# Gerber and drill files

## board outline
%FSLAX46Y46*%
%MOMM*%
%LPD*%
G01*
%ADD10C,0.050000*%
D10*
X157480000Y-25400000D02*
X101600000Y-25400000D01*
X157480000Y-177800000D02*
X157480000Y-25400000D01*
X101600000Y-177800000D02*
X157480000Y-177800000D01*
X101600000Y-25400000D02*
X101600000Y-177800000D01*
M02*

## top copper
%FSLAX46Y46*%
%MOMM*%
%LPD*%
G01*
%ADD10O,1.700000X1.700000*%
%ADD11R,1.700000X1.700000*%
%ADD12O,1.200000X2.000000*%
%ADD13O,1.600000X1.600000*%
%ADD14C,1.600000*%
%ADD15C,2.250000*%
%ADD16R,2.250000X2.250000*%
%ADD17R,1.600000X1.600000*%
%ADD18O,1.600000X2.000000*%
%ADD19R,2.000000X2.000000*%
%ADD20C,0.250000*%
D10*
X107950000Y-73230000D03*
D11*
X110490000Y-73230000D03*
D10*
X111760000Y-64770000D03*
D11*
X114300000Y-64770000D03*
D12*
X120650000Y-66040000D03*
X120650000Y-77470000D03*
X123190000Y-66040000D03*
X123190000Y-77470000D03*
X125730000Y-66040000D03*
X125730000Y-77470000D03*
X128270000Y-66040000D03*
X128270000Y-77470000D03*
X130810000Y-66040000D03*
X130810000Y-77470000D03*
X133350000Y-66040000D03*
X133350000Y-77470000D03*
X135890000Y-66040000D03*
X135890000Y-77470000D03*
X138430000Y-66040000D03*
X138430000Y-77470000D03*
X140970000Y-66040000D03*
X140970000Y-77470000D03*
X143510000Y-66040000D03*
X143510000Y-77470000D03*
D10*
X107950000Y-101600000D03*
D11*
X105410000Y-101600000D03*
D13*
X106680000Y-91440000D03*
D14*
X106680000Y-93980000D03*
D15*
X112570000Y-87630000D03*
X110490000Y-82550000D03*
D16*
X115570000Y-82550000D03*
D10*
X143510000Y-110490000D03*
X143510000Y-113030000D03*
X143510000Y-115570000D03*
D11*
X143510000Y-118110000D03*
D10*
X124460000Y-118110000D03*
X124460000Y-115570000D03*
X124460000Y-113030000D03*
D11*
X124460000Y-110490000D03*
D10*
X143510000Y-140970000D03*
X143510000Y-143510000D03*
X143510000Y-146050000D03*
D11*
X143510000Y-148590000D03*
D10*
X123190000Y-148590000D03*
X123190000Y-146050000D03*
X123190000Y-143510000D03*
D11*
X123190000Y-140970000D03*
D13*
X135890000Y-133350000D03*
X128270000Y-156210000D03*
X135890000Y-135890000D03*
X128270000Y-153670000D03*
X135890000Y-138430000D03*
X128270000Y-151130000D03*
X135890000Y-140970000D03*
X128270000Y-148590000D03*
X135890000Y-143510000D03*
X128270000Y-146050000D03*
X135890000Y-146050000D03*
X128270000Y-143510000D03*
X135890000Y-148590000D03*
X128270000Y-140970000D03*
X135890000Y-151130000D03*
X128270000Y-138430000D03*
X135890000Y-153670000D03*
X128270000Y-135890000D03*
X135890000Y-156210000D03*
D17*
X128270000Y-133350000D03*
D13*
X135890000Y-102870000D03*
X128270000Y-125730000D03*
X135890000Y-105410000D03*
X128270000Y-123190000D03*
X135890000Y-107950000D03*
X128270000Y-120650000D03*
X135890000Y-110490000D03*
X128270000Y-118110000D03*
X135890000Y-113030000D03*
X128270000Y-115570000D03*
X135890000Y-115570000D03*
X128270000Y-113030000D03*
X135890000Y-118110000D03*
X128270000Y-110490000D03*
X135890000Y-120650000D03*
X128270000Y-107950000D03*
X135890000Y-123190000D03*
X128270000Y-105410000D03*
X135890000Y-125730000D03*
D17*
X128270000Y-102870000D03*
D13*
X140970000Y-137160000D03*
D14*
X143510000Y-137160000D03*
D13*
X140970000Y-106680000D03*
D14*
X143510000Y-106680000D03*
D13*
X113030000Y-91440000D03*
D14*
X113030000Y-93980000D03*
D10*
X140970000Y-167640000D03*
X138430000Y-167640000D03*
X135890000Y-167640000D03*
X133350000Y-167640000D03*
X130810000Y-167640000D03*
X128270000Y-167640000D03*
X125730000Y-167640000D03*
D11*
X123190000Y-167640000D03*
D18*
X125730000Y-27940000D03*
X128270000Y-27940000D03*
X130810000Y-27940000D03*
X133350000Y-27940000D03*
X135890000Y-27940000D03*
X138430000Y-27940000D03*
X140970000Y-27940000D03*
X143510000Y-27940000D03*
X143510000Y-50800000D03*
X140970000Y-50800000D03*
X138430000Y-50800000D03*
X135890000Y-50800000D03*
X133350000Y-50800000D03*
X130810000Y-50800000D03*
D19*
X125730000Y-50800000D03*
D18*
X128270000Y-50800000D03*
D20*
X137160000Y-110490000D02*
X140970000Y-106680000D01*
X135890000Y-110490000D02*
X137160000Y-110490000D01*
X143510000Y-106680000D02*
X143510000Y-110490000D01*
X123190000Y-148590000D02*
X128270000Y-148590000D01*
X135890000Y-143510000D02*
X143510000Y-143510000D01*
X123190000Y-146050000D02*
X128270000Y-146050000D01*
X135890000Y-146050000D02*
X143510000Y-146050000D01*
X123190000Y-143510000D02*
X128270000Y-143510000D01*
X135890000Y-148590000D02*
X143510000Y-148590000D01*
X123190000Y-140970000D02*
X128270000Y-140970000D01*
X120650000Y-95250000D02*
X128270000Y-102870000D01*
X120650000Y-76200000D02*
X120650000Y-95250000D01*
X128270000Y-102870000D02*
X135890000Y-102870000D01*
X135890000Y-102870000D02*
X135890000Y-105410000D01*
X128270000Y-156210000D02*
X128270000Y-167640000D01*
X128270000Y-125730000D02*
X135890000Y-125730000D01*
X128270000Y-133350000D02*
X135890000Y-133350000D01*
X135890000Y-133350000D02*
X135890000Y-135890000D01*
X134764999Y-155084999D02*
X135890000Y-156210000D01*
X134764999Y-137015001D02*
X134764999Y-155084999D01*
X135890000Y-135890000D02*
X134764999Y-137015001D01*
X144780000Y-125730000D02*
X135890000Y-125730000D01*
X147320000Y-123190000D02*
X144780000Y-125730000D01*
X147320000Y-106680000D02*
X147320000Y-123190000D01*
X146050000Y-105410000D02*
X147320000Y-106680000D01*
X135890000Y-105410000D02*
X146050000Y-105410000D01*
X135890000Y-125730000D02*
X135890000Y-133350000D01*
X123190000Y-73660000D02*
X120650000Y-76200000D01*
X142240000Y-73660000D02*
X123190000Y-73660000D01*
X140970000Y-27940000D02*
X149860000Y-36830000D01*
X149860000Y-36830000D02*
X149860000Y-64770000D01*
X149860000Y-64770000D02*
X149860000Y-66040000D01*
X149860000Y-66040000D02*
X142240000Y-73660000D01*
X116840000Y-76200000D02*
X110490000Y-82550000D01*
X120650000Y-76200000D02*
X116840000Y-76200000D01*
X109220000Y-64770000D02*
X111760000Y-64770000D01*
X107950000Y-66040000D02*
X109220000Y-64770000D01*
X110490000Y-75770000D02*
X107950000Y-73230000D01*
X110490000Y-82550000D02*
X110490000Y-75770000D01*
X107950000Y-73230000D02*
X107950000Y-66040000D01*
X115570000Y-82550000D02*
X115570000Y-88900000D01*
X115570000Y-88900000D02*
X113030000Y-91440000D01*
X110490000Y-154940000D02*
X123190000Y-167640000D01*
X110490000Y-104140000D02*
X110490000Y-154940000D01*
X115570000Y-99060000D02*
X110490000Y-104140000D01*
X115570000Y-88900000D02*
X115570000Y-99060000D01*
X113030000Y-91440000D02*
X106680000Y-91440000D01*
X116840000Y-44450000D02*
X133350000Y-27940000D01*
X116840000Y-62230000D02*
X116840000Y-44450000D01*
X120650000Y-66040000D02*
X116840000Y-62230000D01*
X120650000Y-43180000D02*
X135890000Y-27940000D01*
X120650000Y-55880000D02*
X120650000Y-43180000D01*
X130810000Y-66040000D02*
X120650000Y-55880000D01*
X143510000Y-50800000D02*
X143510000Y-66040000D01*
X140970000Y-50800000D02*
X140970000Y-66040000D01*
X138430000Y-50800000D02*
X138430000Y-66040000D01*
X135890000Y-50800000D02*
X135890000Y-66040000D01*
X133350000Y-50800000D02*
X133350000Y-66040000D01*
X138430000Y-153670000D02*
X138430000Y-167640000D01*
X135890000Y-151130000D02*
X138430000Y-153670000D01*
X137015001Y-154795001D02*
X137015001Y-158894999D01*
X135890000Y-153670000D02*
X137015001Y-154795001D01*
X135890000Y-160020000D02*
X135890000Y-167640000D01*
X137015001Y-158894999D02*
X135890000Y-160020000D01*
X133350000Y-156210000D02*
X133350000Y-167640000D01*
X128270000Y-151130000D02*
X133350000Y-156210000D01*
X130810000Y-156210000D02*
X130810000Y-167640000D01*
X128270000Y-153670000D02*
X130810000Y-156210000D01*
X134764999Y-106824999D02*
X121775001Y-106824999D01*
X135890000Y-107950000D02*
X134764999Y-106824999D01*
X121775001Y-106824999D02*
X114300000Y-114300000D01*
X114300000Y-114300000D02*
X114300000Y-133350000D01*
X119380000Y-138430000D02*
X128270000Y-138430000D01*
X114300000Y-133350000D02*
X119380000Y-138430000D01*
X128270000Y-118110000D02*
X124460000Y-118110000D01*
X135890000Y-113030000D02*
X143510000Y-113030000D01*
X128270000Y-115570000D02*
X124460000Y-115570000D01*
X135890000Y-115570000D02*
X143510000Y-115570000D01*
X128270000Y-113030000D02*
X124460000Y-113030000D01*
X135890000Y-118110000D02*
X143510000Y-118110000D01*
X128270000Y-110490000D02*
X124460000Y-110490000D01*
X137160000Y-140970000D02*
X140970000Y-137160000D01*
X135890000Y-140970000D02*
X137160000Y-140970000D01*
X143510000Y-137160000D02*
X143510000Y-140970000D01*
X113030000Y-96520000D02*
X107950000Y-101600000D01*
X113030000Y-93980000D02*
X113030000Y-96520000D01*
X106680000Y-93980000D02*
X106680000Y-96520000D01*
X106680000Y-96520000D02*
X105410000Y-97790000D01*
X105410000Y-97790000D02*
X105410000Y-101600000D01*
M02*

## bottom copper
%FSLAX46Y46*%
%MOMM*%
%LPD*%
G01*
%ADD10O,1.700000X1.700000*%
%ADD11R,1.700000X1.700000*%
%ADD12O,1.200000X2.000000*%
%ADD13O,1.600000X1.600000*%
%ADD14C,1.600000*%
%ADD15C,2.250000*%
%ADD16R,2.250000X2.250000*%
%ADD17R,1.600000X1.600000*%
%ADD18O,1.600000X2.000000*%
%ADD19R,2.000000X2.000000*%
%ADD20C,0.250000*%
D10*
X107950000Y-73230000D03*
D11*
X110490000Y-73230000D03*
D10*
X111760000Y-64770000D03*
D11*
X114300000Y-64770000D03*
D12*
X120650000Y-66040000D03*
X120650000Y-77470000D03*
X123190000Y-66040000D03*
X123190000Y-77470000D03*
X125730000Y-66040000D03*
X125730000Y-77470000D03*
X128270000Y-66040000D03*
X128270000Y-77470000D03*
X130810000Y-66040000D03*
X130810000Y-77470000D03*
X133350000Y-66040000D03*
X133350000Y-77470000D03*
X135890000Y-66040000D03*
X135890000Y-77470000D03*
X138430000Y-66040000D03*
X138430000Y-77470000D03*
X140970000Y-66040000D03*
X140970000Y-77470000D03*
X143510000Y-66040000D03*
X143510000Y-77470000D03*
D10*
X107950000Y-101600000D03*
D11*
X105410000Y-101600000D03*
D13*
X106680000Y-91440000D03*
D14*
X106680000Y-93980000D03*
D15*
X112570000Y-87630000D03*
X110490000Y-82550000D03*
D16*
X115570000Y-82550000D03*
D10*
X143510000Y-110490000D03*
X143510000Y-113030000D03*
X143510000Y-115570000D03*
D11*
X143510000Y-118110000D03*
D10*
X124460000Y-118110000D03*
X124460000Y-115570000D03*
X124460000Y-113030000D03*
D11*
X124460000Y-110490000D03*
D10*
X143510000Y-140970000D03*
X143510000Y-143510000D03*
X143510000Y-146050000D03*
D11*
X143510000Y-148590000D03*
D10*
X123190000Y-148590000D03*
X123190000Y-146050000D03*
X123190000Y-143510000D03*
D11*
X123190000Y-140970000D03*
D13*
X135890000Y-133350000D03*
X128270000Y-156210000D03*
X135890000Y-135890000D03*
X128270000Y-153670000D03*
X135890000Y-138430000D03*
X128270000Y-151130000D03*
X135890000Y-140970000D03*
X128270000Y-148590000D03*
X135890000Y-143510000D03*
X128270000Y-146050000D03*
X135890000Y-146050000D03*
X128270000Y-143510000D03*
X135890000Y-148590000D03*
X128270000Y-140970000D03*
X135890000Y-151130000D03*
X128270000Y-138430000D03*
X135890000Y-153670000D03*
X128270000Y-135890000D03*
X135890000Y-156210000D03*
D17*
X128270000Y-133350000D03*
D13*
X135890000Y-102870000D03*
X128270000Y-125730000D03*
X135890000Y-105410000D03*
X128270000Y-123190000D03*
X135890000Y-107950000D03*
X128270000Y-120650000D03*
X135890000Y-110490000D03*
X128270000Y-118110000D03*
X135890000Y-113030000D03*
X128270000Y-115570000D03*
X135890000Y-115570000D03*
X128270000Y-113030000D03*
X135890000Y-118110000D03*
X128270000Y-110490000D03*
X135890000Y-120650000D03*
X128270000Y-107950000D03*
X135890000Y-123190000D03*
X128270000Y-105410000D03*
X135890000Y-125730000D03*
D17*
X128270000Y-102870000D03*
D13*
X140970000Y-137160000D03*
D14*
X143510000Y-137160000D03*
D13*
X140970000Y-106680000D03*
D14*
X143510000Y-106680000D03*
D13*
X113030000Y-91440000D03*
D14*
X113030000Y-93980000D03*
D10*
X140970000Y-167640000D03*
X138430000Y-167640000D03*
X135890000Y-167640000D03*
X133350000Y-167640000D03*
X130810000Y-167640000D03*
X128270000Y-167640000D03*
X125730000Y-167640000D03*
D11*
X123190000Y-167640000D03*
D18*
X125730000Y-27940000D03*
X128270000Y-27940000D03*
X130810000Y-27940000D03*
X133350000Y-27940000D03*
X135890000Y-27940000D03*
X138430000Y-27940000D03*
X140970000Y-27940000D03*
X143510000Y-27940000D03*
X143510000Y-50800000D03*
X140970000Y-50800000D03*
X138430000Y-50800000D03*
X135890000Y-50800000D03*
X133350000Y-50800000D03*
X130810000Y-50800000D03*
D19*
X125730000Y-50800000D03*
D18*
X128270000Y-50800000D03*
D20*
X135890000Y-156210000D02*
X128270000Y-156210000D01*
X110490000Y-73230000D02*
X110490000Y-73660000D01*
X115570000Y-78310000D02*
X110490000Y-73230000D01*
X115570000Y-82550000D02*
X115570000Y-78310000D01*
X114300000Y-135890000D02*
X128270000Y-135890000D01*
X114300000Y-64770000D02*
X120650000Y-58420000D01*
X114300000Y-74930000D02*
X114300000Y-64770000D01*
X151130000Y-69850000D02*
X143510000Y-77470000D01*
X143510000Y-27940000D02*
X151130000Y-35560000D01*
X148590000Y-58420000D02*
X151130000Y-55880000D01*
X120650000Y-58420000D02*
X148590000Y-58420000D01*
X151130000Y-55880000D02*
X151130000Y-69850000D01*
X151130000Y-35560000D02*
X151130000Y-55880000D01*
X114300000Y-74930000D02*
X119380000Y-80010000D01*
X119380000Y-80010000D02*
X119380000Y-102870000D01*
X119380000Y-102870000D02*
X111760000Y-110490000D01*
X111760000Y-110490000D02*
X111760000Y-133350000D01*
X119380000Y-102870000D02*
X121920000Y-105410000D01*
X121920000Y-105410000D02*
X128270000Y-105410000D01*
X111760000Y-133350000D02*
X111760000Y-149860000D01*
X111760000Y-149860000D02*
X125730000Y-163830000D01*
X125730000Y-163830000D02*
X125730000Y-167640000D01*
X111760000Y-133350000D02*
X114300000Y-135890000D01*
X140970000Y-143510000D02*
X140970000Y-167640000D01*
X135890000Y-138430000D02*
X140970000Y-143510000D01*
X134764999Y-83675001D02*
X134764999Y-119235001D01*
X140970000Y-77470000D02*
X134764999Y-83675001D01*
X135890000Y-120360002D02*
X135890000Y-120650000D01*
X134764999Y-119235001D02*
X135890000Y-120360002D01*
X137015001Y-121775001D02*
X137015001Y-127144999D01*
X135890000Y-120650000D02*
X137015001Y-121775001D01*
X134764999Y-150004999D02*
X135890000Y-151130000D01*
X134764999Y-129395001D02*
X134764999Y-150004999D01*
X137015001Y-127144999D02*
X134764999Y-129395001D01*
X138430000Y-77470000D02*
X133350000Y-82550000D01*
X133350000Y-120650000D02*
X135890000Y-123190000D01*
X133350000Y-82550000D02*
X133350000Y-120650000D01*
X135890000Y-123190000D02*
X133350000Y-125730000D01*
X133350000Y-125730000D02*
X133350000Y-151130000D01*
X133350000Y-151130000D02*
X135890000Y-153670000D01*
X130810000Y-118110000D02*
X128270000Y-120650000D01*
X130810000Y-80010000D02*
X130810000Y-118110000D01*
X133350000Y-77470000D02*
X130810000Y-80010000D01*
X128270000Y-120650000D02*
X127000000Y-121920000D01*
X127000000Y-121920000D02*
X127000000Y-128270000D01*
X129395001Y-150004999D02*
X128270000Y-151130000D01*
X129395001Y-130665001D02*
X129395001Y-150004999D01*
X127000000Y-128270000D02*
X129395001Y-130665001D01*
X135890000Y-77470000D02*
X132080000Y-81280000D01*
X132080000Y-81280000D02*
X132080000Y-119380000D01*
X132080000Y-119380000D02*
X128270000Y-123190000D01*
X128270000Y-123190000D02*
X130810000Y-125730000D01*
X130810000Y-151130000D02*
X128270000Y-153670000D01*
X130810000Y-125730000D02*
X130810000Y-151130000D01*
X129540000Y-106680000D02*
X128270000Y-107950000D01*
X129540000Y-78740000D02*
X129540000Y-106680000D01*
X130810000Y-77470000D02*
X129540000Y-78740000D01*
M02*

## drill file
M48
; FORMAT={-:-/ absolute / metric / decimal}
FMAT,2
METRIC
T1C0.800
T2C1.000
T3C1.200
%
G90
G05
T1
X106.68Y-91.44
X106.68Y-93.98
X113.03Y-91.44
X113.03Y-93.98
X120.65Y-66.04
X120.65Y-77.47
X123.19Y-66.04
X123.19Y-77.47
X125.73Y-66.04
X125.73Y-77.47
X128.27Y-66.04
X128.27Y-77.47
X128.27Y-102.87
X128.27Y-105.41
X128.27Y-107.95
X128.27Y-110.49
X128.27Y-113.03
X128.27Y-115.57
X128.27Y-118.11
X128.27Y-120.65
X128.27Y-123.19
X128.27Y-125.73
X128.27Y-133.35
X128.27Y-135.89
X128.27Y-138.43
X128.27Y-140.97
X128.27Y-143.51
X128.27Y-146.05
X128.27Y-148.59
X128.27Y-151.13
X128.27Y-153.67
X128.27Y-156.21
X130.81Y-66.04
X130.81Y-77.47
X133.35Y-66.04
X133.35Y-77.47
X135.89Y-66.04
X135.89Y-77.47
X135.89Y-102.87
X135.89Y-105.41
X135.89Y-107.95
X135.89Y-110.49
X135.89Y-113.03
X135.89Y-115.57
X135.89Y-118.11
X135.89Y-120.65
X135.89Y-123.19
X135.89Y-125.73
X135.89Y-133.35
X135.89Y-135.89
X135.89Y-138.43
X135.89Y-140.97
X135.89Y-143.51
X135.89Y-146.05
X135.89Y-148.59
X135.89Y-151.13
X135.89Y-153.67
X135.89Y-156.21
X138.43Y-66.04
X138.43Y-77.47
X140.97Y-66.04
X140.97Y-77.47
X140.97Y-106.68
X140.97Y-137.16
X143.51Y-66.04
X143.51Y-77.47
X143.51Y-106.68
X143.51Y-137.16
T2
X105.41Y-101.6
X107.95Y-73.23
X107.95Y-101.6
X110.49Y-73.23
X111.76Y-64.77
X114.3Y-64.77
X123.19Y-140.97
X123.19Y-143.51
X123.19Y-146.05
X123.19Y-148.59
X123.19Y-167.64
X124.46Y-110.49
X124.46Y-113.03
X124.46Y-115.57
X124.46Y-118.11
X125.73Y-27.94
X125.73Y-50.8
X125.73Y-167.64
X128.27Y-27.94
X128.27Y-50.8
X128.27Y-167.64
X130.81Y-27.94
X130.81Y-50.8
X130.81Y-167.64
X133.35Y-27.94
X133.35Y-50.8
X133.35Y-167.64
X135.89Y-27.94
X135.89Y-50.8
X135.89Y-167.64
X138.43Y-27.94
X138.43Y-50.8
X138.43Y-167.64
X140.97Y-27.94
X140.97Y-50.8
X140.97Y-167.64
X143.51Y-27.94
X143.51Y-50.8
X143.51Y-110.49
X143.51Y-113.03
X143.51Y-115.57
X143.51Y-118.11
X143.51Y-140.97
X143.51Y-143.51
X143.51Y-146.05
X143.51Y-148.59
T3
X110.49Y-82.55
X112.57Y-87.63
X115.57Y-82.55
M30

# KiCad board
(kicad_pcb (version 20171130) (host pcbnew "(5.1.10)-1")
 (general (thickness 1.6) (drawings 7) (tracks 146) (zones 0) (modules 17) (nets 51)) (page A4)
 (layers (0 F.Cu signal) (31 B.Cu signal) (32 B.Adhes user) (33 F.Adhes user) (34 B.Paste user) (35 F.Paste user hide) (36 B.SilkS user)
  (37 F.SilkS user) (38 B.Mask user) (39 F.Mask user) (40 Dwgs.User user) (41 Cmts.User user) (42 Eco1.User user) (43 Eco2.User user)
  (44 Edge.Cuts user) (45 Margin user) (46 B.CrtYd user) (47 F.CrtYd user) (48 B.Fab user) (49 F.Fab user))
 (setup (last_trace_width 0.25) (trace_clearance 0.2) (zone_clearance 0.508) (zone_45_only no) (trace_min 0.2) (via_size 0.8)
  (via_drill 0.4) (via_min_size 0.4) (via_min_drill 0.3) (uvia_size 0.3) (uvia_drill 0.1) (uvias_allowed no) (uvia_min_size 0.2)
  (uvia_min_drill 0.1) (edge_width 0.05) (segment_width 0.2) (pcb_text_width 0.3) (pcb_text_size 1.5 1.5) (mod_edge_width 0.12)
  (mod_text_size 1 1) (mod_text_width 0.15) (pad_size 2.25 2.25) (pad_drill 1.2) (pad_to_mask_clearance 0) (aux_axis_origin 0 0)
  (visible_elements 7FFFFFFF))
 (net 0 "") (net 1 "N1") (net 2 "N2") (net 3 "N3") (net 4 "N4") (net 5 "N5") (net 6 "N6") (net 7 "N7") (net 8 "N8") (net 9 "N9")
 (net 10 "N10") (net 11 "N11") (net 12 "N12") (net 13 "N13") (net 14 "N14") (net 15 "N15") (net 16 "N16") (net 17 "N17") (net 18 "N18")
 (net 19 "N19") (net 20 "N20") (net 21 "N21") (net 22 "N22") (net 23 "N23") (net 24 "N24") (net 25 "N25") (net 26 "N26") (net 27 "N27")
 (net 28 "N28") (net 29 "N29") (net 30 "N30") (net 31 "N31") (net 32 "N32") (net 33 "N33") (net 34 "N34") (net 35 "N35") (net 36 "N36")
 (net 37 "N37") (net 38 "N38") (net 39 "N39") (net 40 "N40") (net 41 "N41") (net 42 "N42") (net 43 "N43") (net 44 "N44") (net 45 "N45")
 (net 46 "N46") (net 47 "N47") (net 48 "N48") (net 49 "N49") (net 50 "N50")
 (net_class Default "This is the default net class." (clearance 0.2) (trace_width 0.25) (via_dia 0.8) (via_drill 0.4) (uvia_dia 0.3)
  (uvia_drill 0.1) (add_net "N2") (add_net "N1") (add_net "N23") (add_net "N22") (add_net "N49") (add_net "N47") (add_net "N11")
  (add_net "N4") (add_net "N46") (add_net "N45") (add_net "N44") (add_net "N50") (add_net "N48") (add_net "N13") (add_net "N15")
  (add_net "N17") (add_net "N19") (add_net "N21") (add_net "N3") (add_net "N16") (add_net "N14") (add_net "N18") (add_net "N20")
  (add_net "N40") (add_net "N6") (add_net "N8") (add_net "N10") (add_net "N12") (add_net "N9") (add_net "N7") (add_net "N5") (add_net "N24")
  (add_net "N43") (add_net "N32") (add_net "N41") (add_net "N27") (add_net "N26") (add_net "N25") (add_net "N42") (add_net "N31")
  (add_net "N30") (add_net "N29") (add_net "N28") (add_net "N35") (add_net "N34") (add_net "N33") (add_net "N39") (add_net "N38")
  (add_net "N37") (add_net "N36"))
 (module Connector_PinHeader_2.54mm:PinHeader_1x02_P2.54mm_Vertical (layer F.Cu) (at 110.49 73.23 270)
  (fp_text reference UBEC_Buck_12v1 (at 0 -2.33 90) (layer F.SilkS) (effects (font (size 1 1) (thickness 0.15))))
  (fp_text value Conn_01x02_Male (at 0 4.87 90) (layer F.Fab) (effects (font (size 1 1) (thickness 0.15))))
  (pad 2 thru_hole oval (at 0 2.54 270) (size 1.7 1.7) (drill 1) (layers *.Cu *.Mask) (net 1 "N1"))
  (pad 1 thru_hole rect (at 0 0 270) (size 1.7 1.7) (drill 1) (layers *.Cu *.Mask) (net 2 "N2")))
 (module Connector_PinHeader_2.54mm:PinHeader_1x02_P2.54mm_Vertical (layer F.Cu) (at 114.3 64.77 270)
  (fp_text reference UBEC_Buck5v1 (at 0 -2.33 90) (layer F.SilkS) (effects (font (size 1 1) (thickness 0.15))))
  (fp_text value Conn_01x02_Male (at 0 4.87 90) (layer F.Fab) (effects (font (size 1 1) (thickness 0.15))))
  (pad 2 thru_hole oval (at 0 2.54 270) (size 1.7 1.7) (drill 1) (layers *.Cu *.Mask) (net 1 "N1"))
  (pad 1 thru_hole rect (at 0 0 270) (size 1.7 1.7) (drill 1) (layers *.Cu *.Mask) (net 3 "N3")))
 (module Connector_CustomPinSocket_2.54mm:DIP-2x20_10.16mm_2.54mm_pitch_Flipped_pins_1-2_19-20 (layer F.Cu) (at 132.08 64.77 270)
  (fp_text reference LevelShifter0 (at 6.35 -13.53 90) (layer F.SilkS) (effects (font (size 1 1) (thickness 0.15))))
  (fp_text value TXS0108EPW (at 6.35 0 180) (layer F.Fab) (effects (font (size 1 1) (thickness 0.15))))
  (pad 10 thru_hole oval (at 1.27 11.43 180) (size 1.2 2) (drill 0.8) (layers *.Cu *.Mask) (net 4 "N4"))
  (pad 11 thru_hole oval (at 12.7 11.43 180) (size 1.2 2) (drill 0.8) (layers *.Cu *.Mask) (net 1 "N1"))
  (pad 9 thru_hole oval (at 1.27 8.89 180) (size 1.2 2) (drill 0.8) (layers *.Cu *.Mask) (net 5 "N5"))
  (pad 12 thru_hole oval (at 12.7 8.89 180) (size 1.2 2) (drill 0.8) (layers *.Cu *.Mask) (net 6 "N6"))
  (pad 8 thru_hole oval (at 1.27 6.35 180) (size 1.2 2) (drill 0.8) (layers *.Cu *.Mask) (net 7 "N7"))
  (pad 13 thru_hole oval (at 12.7 6.35 180) (size 1.2 2) (drill 0.8) (layers *.Cu *.Mask) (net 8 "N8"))
  (pad 7 thru_hole oval (at 1.27 3.81 180) (size 1.2 2) (drill 0.8) (layers *.Cu *.Mask) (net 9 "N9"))
  (pad 14 thru_hole oval (at 12.7 3.81 180) (size 1.2 2) (drill 0.8) (layers *.Cu *.Mask) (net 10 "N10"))
  (pad 6 thru_hole oval (at 1.27 1.27 180) (size 1.2 2) (drill 0.8) (layers *.Cu *.Mask) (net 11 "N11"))
  (pad 15 thru_hole oval (at 12.7 1.27 180) (size 1.2 2) (drill 0.8) (layers *.Cu *.Mask) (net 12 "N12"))
  (pad 5 thru_hole oval (at 1.27 -1.27 180) (size 1.2 2) (drill 0.8) (layers *.Cu *.Mask) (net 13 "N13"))
  (pad 16 thru_hole oval (at 12.7 -1.27 180) (size 1.2 2) (drill 0.8) (layers *.Cu *.Mask) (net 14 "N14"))
  (pad 4 thru_hole oval (at 1.27 -3.81 180) (size 1.2 2) (drill 0.8) (layers *.Cu *.Mask) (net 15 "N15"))
  (pad 17 thru_hole oval (at 12.7 -3.81 180) (size 1.2 2) (drill 0.8) (layers *.Cu *.Mask) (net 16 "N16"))
  (pad 3 thru_hole oval (at 1.27 -6.35 180) (size 1.2 2) (drill 0.8) (layers *.Cu *.Mask) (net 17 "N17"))
  (pad 18 thru_hole oval (at 12.7 -6.35 180) (size 1.2 2) (drill 0.8) (layers *.Cu *.Mask) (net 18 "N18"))
  (pad 1 thru_hole oval (at 1.27 -8.89 180) (size 1.2 2) (drill 0.8) (layers *.Cu *.Mask) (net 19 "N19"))
  (pad 20 thru_hole oval (at 12.7 -8.89 180) (size 1.2 2) (drill 0.8) (layers *.Cu *.Mask) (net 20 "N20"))
  (pad 2 thru_hole oval (at 1.27 -11.43 180) (size 1.2 2) (drill 0.8) (layers *.Cu *.Mask) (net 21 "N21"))
  (pad 19 thru_hole oval (at 12.7 -11.43 180) (size 1.2 2) (drill 0.8) (layers *.Cu *.Mask) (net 3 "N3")))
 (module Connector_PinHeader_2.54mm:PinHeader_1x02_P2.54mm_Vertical (layer F.Cu) (at 105.41 101.6 90)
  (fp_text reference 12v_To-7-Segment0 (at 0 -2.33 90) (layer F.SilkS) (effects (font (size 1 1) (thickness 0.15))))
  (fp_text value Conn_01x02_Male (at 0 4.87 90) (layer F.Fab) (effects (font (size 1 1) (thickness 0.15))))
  (pad 2 thru_hole oval (at 0 2.54 90) (size 1.7 1.7) (drill 1) (layers *.Cu *.Mask) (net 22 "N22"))
  (pad 1 thru_hole rect (at 0 0 90) (size 1.7 1.7) (drill 1) (layers *.Cu *.Mask) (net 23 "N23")))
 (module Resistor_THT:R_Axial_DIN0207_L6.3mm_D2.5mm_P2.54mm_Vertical (layer F.Cu) (at 106.68 93.98 90)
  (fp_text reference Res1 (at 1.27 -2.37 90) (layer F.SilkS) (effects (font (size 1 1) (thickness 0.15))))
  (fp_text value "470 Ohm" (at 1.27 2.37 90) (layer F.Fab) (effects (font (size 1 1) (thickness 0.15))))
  (pad 2 thru_hole oval (at 2.54 0 90) (size 1.6 1.6) (drill 0.8) (layers *.Cu *.Mask) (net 2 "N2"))
  (pad 1 thru_hole circle (at 0 0 90) (size 1.6 1.6) (drill 0.8) (layers *.Cu *.Mask) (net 23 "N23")))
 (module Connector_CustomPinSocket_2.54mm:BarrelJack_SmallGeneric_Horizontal (layer F.Cu) (at 115.57 82.55 270)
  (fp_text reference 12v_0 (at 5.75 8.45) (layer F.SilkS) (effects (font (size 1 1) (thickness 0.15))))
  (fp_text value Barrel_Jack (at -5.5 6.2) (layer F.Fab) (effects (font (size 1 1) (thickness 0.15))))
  (pad 3 thru_hole circle (at 5.08 3 270) (size 2.25 2.25) (drill 1.2) (layers *.Cu *.Mask))
  (pad 2 thru_hole circle (at 0 5.08 270) (size 2.25 2.25) (drill 1.2) (layers *.Cu *.Mask) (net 1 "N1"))
  (pad 1 thru_hole rect (at 0 0 270) (size 2.25 2.25) (drill 1.2) (layers *.Cu *.Mask) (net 2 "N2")))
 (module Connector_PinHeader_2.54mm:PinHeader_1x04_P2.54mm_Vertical (layer F.Cu) (at 143.51 118.11 180)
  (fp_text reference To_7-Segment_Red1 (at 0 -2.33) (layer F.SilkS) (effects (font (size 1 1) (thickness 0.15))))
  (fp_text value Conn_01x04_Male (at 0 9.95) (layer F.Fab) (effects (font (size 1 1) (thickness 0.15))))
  (pad 4 thru_hole oval (at 0 7.62 180) (size 1.7 1.7) (drill 1) (layers *.Cu *.Mask) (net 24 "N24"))
  (pad 3 thru_hole oval (at 0 5.08 180) (size 1.7 1.7) (drill 1) (layers *.Cu *.Mask) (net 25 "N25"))
  (pad 2 thru_hole oval (at 0 2.54 180) (size 1.7 1.7) (drill 1) (layers *.Cu *.Mask) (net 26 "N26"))
  (pad 1 thru_hole rect (at 0 0 180) (size 1.7 1.7) (drill 1) (layers *.Cu *.Mask) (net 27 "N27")))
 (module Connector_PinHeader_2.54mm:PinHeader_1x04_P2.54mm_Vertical (layer F.Cu) (at 124.46 110.49)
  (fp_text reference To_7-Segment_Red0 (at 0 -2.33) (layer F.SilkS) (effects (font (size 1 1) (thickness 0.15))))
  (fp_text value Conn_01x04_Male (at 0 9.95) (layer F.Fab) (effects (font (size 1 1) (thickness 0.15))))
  (pad 4 thru_hole oval (at 0 7.62) (size 1.7 1.7) (drill 1) (layers *.Cu *.Mask) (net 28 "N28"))
  (pad 3 thru_hole oval (at 0 5.08) (size 1.7 1.7) (drill 1) (layers *.Cu *.Mask) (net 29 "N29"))
  (pad 2 thru_hole oval (at 0 2.54) (size 1.7 1.7) (drill 1) (layers *.Cu *.Mask) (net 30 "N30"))
  (pad 1 thru_hole rect (at 0 0) (size 1.7 1.7) (drill 1) (layers *.Cu *.Mask) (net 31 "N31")))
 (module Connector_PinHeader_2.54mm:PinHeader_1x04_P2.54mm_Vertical (layer F.Cu) (at 143.51 148.59 180)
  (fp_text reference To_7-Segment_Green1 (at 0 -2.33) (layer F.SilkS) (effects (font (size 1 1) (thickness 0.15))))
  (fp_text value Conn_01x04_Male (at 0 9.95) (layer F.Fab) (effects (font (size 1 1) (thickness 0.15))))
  (pad 4 thru_hole oval (at 0 7.62 180) (size 1.7 1.7) (drill 1) (layers *.Cu *.Mask) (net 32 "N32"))
  (pad 3 thru_hole oval (at 0 5.08 180) (size 1.7 1.7) (drill 1) (layers *.Cu *.Mask) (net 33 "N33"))
  (pad 2 thru_hole oval (at 0 2.54 180) (size 1.7 1.7) (drill 1) (layers *.Cu *.Mask) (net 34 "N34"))
  (pad 1 thru_hole rect (at 0 0 180) (size 1.7 1.7) (drill 1) (layers *.Cu *.Mask) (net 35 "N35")))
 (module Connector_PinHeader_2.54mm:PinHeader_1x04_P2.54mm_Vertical (layer F.Cu) (at 123.19 140.97)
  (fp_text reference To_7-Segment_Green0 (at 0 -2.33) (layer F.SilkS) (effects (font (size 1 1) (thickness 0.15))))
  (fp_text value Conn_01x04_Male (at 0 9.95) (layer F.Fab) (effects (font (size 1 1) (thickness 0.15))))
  (pad 4 thru_hole oval (at 0 7.62) (size 1.7 1.7) (drill 1) (layers *.Cu *.Mask) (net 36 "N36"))
  (pad 3 thru_hole oval (at 0 5.08) (size 1.7 1.7) (drill 1) (layers *.Cu *.Mask) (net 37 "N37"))
  (pad 2 thru_hole oval (at 0 2.54) (size 1.7 1.7) (drill 1) (layers *.Cu *.Mask) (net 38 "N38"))
  (pad 1 thru_hole rect (at 0 0) (size 1.7 1.7) (drill 1) (layers *.Cu *.Mask) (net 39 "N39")))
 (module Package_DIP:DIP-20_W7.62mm (layer F.Cu) (at 128.27 133.35)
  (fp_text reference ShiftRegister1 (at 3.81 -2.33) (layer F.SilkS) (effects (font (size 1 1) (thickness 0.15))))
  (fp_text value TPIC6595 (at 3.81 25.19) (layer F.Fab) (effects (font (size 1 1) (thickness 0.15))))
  (pad 20 thru_hole oval (at 7.62 0) (size 1.6 1.6) (drill 0.8) (layers *.Cu *.Mask) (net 1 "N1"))
  (pad 10 thru_hole oval (at 0 22.86) (size 1.6 1.6) (drill 0.8) (layers *.Cu *.Mask) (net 1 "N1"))
  (pad 19 thru_hole oval (at 7.62 2.54) (size 1.6 1.6) (drill 0.8) (layers *.Cu *.Mask) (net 1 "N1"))
  (pad 9 thru_hole oval (at 0 20.32) (size 1.6 1.6) (drill 0.8) (layers *.Cu *.Mask) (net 16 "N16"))
  (pad 18 thru_hole oval (at 7.62 5.08) (size 1.6 1.6) (drill 0.8) (layers *.Cu *.Mask) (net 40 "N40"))
  (pad 8 thru_hole oval (at 0 17.78) (size 1.6 1.6) (drill 0.8) (layers *.Cu *.Mask) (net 14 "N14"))
  (pad 17 thru_hole oval (at 7.62 7.62) (size 1.6 1.6) (drill 0.8) (layers *.Cu *.Mask) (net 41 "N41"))
  (pad 7 thru_hole oval (at 0 15.24) (size 1.6 1.6) (drill 0.8) (layers *.Cu *.Mask) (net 36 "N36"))
  (pad 16 thru_hole oval (at 7.62 10.16) (size 1.6 1.6) (drill 0.8) (layers *.Cu *.Mask) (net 33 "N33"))
  (pad 6 thru_hole oval (at 0 12.7) (size 1.6 1.6) (drill 0.8) (layers *.Cu *.Mask) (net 37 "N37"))
  (pad 15 thru_hole oval (at 7.62 12.7) (size 1.6 1.6) (drill 0.8) (layers *.Cu *.Mask) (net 34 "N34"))
  (pad 5 thru_hole oval (at 0 10.16) (size 1.6 1.6) (drill 0.8) (layers *.Cu *.Mask) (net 38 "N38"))
  (pad 14 thru_hole oval (at 7.62 15.24) (size 1.6 1.6) (drill 0.8) (layers *.Cu *.Mask) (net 35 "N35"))
  (pad 4 thru_hole oval (at 0 7.62) (size 1.6 1.6) (drill 0.8) (layers *.Cu *.Mask) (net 39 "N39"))
  (pad 13 thru_hole oval (at 7.62 17.78) (size 1.6 1.6) (drill 0.8) (layers *.Cu *.Mask) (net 20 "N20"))
  (pad 3 thru_hole oval (at 0 5.08) (size 1.6 1.6) (drill 0.8) (layers *.Cu *.Mask) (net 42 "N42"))
  (pad 12 thru_hole oval (at 7.62 20.32) (size 1.6 1.6) (drill 0.8) (layers *.Cu *.Mask) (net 18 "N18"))
  (pad 2 thru_hole oval (at 0 2.54) (size 1.6 1.6) (drill 0.8) (layers *.Cu *.Mask) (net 3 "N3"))
  (pad 11 thru_hole oval (at 7.62 22.86) (size 1.6 1.6) (drill 0.8) (layers *.Cu *.Mask) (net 1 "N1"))
  (pad 1 thru_hole rect (at 0 0) (size 1.6 1.6) (drill 0.8) (layers *.Cu *.Mask) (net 1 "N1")))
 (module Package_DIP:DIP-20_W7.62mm (layer F.Cu) (at 128.27 102.87)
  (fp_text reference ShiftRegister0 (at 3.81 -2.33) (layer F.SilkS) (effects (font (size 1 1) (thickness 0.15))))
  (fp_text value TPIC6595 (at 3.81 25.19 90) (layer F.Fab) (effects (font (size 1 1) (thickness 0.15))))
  (pad 20 thru_hole oval (at 7.62 0) (size 1.6 1.6) (drill 0.8) (layers *.Cu *.Mask) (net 1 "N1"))
  (pad 10 thru_hole oval (at 0 22.86) (size 1.6 1.6) (drill 0.8) (layers *.Cu *.Mask) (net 1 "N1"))
  (pad 19 thru_hole oval (at 7.62 2.54) (size 1.6 1.6) (drill 0.8) (layers *.Cu *.Mask) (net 1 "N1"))
  (pad 9 thru_hole oval (at 0 20.32) (size 1.6 1.6) (drill 0.8) (layers *.Cu *.Mask) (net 16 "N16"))
  (pad 18 thru_hole oval (at 7.62 5.08) (size 1.6 1.6) (drill 0.8) (layers *.Cu *.Mask) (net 42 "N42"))
  (pad 8 thru_hole oval (at 0 17.78) (size 1.6 1.6) (drill 0.8) (layers *.Cu *.Mask) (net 14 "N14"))
  (pad 17 thru_hole oval (at 7.62 7.62) (size 1.6 1.6) (drill 0.8) (layers *.Cu *.Mask) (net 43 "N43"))
  (pad 7 thru_hole oval (at 0 15.24) (size 1.6 1.6) (drill 0.8) (layers *.Cu *.Mask) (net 28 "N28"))
  (pad 16 thru_hole oval (at 7.62 10.16) (size 1.6 1.6) (drill 0.8) (layers *.Cu *.Mask) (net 25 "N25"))
  (pad 6 thru_hole oval (at 0 12.7) (size 1.6 1.6) (drill 0.8) (layers *.Cu *.Mask) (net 29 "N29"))
  (pad 15 thru_hole oval (at 7.62 12.7) (size 1.6 1.6) (drill 0.8) (layers *.Cu *.Mask) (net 26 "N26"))
  (pad 5 thru_hole oval (at 0 10.16) (size 1.6 1.6) (drill 0.8) (layers *.Cu *.Mask) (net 30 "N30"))
  (pad 14 thru_hole oval (at 7.62 15.24) (size 1.6 1.6) (drill 0.8) (layers *.Cu *.Mask) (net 27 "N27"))
  (pad 4 thru_hole oval (at 0 7.62) (size 1.6 1.6) (drill 0.8) (layers *.Cu *.Mask) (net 31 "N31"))
  (pad 13 thru_hole oval (at 7.62 17.78) (size 1.6 1.6) (drill 0.8) (layers *.Cu *.Mask) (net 20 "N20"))
  (pad 3 thru_hole oval (at 0 5.08) (size 1.6 1.6) (drill 0.8) (layers *.Cu *.Mask) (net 12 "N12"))
  (pad 12 thru_hole oval (at 7.62 20.32) (size 1.6 1.6) (drill 0.8) (layers *.Cu *.Mask) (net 18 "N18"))
  (pad 2 thru_hole oval (at 0 2.54) (size 1.6 1.6) (drill 0.8) (layers *.Cu *.Mask) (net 3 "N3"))
  (pad 11 thru_hole oval (at 7.62 22.86) (size 1.6 1.6) (drill 0.8) (layers *.Cu *.Mask) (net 1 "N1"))
  (pad 1 thru_hole rect (at 0 0) (size 1.6 1.6) (drill 0.8) (layers *.Cu *.Mask) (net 1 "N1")))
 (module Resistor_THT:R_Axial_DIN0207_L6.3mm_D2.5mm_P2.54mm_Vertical (layer F.Cu) (at 143.51 137.16 180)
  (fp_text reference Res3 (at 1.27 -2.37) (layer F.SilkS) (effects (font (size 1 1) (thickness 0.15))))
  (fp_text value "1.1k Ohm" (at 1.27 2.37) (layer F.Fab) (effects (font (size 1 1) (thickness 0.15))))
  (pad 2 thru_hole oval (at 2.54 0 180) (size 1.6 1.6) (drill 0.8) (layers *.Cu *.Mask) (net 41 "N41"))
  (pad 1 thru_hole circle (at 0 0 180) (size 1.6 1.6) (drill 0.8) (layers *.Cu *.Mask) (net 32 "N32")))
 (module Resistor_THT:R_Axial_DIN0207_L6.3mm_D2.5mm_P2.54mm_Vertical (layer F.Cu) (at 143.51 106.68 180)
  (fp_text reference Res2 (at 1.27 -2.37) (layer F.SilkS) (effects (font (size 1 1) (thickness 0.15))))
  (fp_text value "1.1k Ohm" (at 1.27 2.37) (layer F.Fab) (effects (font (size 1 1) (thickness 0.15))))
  (pad 2 thru_hole oval (at 2.54 0 180) (size 1.6 1.6) (drill 0.8) (layers *.Cu *.Mask) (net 43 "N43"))
  (pad 1 thru_hole circle (at 0 0 180) (size 1.6 1.6) (drill 0.8) (layers *.Cu *.Mask) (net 24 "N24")))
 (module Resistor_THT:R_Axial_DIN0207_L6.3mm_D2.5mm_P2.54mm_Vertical (layer F.Cu) (at 113.03 93.98 90)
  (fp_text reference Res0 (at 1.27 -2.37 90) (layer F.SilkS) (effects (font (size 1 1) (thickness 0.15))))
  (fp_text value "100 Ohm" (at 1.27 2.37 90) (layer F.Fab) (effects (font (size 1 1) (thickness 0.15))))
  (pad 2 thru_hole oval (at 2.54 0 90) (size 1.6 1.6) (drill 0.8) (layers *.Cu *.Mask) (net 2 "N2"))
  (pad 1 thru_hole circle (at 0 0 90) (size 1.6 1.6) (drill 0.8) (layers *.Cu *.Mask) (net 22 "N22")))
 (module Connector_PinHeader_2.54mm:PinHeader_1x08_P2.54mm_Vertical (layer F.Cu) (at 123.19 167.64 90)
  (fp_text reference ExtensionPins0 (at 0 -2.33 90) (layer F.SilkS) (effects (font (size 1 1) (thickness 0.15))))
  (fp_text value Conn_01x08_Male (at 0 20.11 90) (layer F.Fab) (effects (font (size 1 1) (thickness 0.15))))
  (pad 8 thru_hole oval (at 0 17.78 90) (size 1.7 1.7) (drill 1) (layers *.Cu *.Mask) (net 40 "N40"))
  (pad 7 thru_hole oval (at 0 15.24 90) (size 1.7 1.7) (drill 1) (layers *.Cu *.Mask) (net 20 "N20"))
  (pad 6 thru_hole oval (at 0 12.7 90) (size 1.7 1.7) (drill 1) (layers *.Cu *.Mask) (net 18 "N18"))
  (pad 5 thru_hole oval (at 0 10.16 90) (size 1.7 1.7) (drill 1) (layers *.Cu *.Mask) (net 14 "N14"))
  (pad 4 thru_hole oval (at 0 7.62 90) (size 1.7 1.7) (drill 1) (layers *.Cu *.Mask) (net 16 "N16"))
  (pad 3 thru_hole oval (at 0 5.08 90) (size 1.7 1.7) (drill 1) (layers *.Cu *.Mask) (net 1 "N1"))
  (pad 2 thru_hole oval (at 0 2.54 90) (size 1.7 1.7) (drill 1) (layers *.Cu *.Mask) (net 3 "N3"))
  (pad 1 thru_hole rect (at 0 0 90) (size 1.7 1.7) (drill 1) (layers *.Cu *.Mask) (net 2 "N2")))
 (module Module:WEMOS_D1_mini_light (layer F.Cu) (at 125.73 50.8 90)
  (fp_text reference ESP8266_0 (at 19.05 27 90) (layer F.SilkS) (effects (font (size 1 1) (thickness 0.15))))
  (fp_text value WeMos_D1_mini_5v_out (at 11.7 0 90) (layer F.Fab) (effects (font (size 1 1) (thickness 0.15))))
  (pad 16 thru_hole oval (at 22.86 0 90) (size 2 1.6) (drill 1) (layers *.Cu *.Mask) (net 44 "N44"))
  (pad 15 thru_hole oval (at 22.86 2.54 90) (size 2 1.6) (drill 1) (layers *.Cu *.Mask) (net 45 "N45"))
  (pad 14 thru_hole oval (at 22.86 5.08 90) (size 2 1.6) (drill 1) (layers *.Cu *.Mask) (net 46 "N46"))
  (pad 13 thru_hole oval (at 22.86 7.62 90) (size 2 1.6) (drill 1) (layers *.Cu *.Mask) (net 4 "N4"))
  (pad 12 thru_hole oval (at 22.86 10.16 90) (size 2 1.6) (drill 1) (layers *.Cu *.Mask) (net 11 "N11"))
  (pad 11 thru_hole oval (at 22.86 12.7 90) (size 2 1.6) (drill 1) (layers *.Cu *.Mask) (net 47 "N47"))
  (pad 10 thru_hole oval (at 22.86 15.24 90) (size 2 1.6) (drill 1) (layers *.Cu *.Mask) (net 1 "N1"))
  (pad 9 thru_hole oval (at 22.86 17.78 90) (size 2 1.6) (drill 1) (layers *.Cu *.Mask) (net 3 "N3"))
  (pad 8 thru_hole oval (at 0 17.78 90) (size 2 1.6) (drill 1) (layers *.Cu *.Mask) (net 21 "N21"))
  (pad 7 thru_hole oval (at 0 15.24 90) (size 2 1.6) (drill 1) (layers *.Cu *.Mask) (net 19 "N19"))
  (pad 6 thru_hole oval (at 0 12.7 90) (size 2 1.6) (drill 1) (layers *.Cu *.Mask) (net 17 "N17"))
  (pad 5 thru_hole oval (at 0 10.16 90) (size 2 1.6) (drill 1) (layers *.Cu *.Mask) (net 15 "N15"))
  (pad 4 thru_hole oval (at 0 7.62 90) (size 2 1.6) (drill 1) (layers *.Cu *.Mask) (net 13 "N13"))
  (pad 3 thru_hole oval (at 0 5.08 90) (size 2 1.6) (drill 1) (layers *.Cu *.Mask) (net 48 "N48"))
  (pad 1 thru_hole rect (at 0 0 90) (size 2 2) (drill 1) (layers *.Cu *.Mask) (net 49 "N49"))
  (pad 2 thru_hole oval (at 0 2.54 90) (size 2 1.6) (drill 1) (layers *.Cu *.Mask) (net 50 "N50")))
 (gr_line (start 157.48 25.4) (end 101.6 25.4) (layer Edge.Cuts) (width 0.05))
 (gr_line (start 157.48 177.8) (end 157.48 25.4) (layer Edge.Cuts) (width 0.05))
 (gr_line (start 101.6 177.8) (end 157.48 177.8) (layer Edge.Cuts) (width 0.05))
 (gr_line (start 101.6 25.4) (end 101.6 177.8) (layer Edge.Cuts) (width 0.05))
 (segment (start 137.16 110.49) (end 140.97 106.68) (width 0.25) (layer F.Cu) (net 43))
 (segment (start 135.89 110.49) (end 137.16 110.49) (width 0.25) (layer F.Cu) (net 43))
 (segment (start 143.51 106.68) (end 143.51 110.49) (width 0.25) (layer F.Cu) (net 24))
 (segment (start 123.19 148.59) (end 128.27 148.59) (width 0.25) (layer F.Cu) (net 36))
 (segment (start 135.89 143.51) (end 143.51 143.51) (width 0.25) (layer F.Cu) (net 33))
 (segment (start 123.19 146.05) (end 128.27 146.05) (width 0.25) (layer F.Cu) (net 37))
 (segment (start 135.89 146.05) (end 143.51 146.05) (width 0.25) (layer F.Cu) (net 34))
 (segment (start 123.19 143.51) (end 128.27 143.51) (width 0.25) (layer F.Cu) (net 38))
 (segment (start 135.89 148.59) (end 143.51 148.59) (width 0.25) (layer F.Cu) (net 35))
 (segment (start 123.19 140.97) (end 128.27 140.97) (width 0.25) (layer F.Cu) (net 39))
 (segment (start 120.65 95.25) (end 128.27 102.87) (width 0.25) (layer F.Cu) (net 1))
 (segment (start 120.65 76.2) (end 120.65 95.25) (width 0.25) (layer F.Cu) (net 1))
 (segment (start 128.27 102.87) (end 135.89 102.87) (width 0.25) (layer F.Cu) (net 1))
 (segment (start 135.89 102.87) (end 135.89 105.41) (width 0.25) (layer F.Cu) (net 1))
 (segment (start 128.27 156.21) (end 128.27 167.64) (width 0.25) (layer F.Cu) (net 1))
 (segment (start 135.89 156.21) (end 128.27 156.21) (width 0.25) (layer B.Cu) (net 1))
 (segment (start 128.27 125.73) (end 135.89 125.73) (width 0.25) (layer F.Cu) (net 1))
 (segment (start 128.27 133.35) (end 135.89 133.35) (width 0.25) (layer F.Cu) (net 1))
 (segment (start 135.89 133.35) (end 135.89 135.89) (width 0.25) (layer F.Cu) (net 1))
 (segment (start 134.764999 155.084999) (end 135.89 156.21) (width 0.25) (layer F.Cu) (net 1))
 (segment (start 134.764999 137.015001) (end 134.764999 155.084999) (width 0.25) (layer F.Cu) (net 1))
 (segment (start 135.89 135.89) (end 134.764999 137.015001) (width 0.25) (layer F.Cu) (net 1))
 (segment (start 144.78 125.73) (end 135.89 125.73) (width 0.25) (layer F.Cu) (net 1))
 (segment (start 147.32 123.19) (end 144.78 125.73) (width 0.25) (layer F.Cu) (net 1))
 (segment (start 147.32 106.68) (end 147.32 123.19) (width 0.25) (layer F.Cu) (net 1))
 (segment (start 146.05 105.41) (end 147.32 106.68) (width 0.25) (layer F.Cu) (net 1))
 (segment (start 135.89 105.41) (end 146.05 105.41) (width 0.25) (layer F.Cu) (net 1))
 (segment (start 135.89 125.73) (end 135.89 133.35) (width 0.25) (layer F.Cu) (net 1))
 (segment (start 123.19 73.66) (end 120.65 76.2) (width 0.25) (layer F.Cu) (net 1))
 (segment (start 142.24 73.66) (end 123.19 73.66) (width 0.25) (layer F.Cu) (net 1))
 (segment (start 140.97 27.94) (end 149.86 36.83) (width 0.25) (layer F.Cu) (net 1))
 (segment (start 149.86 36.83) (end 149.86 64.77) (width 0.25) (layer F.Cu) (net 1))
 (segment (start 149.86 64.77) (end 149.86 66.04) (width 0.25) (layer F.Cu) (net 1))
 (segment (start 149.86 66.04) (end 142.24 73.66) (width 0.25) (layer F.Cu) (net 1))
 (segment (start 116.84 76.2) (end 110.49 82.55) (width 0.25) (layer F.Cu) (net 1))
 (segment (start 120.65 76.2) (end 116.84 76.2) (width 0.25) (layer F.Cu) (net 1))
 (segment (start 109.22 64.77) (end 111.76 64.77) (width 0.25) (layer F.Cu) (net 1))
 (segment (start 107.95 66.04) (end 109.22 64.77) (width 0.25) (layer F.Cu) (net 1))
 (segment (start 110.49 75.77) (end 107.95 73.23) (width 0.25) (layer F.Cu) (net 1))
 (segment (start 110.49 82.55) (end 110.49 75.77) (width 0.25) (layer F.Cu) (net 1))
 (segment (start 107.95 73.23) (end 107.95 66.04) (width 0.25) (layer F.Cu) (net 1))
 (segment (start 115.57 82.55) (end 115.57 88.9) (width 0.25) (layer F.Cu) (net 2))
 (segment (start 115.57 88.9) (end 113.03 91.44) (width 0.25) (layer F.Cu) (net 2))
 (segment (start 110.49 154.94) (end 123.19 167.64) (width 0.25) (layer F.Cu) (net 2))
 (segment (start 110.49 104.14) (end 110.49 154.94) (width 0.25) (layer F.Cu) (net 2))
 (segment (start 115.57 99.06) (end 110.49 104.14) (width 0.25) (layer F.Cu) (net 2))
 (segment (start 115.57 88.9) (end 115.57 99.06) (width 0.25) (layer F.Cu) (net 2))
 (segment (start 113.03 91.44) (end 106.68 91.44) (width 0.25) (layer F.Cu) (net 2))
 (segment (start 110.49 73.23) (end 110.49 73.66) (width 0.25) (layer B.Cu) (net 2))
 (segment (start 115.57 78.31) (end 110.49 73.23) (width 0.25) (layer B.Cu) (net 2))
 (segment (start 115.57 82.55) (end 115.57 78.31) (width 0.25) (layer B.Cu) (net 2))
 (segment (start 116.84 44.45) (end 133.35 27.94) (width 0.25) (layer F.Cu) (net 4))
 (segment (start 116.84 62.23) (end 116.84 44.45) (width 0.25) (layer F.Cu) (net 4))
 (segment (start 120.65 66.04) (end 116.84 62.23) (width 0.25) (layer F.Cu) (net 4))
 (segment (start 120.65 43.18) (end 135.89 27.94) (width 0.25) (layer F.Cu) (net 11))
 (segment (start 120.65 55.88) (end 120.65 43.18) (width 0.25) (layer F.Cu) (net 11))
 (segment (start 130.81 66.04) (end 120.65 55.88) (width 0.25) (layer F.Cu) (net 11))
 (segment (start 114.3 135.89) (end 128.27 135.89) (width 0.25) (layer B.Cu) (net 3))
 (segment (start 114.3 64.77) (end 120.65 58.42) (width 0.25) (layer B.Cu) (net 3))
 (segment (start 114.3 74.93) (end 114.3 64.77) (width 0.25) (layer B.Cu) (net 3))
 (segment (start 151.13 69.85) (end 143.51 77.47) (width 0.25) (layer B.Cu) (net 3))
 (segment (start 143.51 27.94) (end 151.13 35.56) (width 0.25) (layer B.Cu) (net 3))
 (segment (start 148.59 58.42) (end 151.13 55.88) (width 0.25) (layer B.Cu) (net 3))
 (segment (start 120.65 58.42) (end 148.59 58.42) (width 0.25) (layer B.Cu) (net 3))
 (segment (start 151.13 55.88) (end 151.13 69.85) (width 0.25) (layer B.Cu) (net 3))
 (segment (start 151.13 35.56) (end 151.13 55.88) (width 0.25) (layer B.Cu) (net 3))
 (segment (start 114.3 74.93) (end 119.38 80.01) (width 0.25) (layer B.Cu) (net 3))
 (segment (start 119.38 80.01) (end 119.38 102.87) (width 0.25) (layer B.Cu) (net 3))
 (segment (start 119.38 102.87) (end 111.76 110.49) (width 0.25) (layer B.Cu) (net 3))
 (segment (start 111.76 110.49) (end 111.76 133.35) (width 0.25) (layer B.Cu) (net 3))
 (segment (start 119.38 102.87) (end 121.92 105.41) (width 0.25) (layer B.Cu) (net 3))
 (segment (start 121.92 105.41) (end 128.27 105.41) (width 0.25) (layer B.Cu) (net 3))
 (segment (start 111.76 133.35) (end 111.76 149.86) (width 0.25) (layer B.Cu) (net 3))
 (segment (start 111.76 149.86) (end 125.73 163.83) (width 0.25) (layer B.Cu) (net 3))
 (segment (start 125.73 163.83) (end 125.73 167.64) (width 0.25) (layer B.Cu) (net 3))
 (segment (start 111.76 133.35) (end 114.3 135.89) (width 0.25) (layer B.Cu) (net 3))
 (segment (start 143.51 50.8) (end 143.51 66.04) (width 0.25) (layer F.Cu) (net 21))
 (segment (start 140.97 50.8) (end 140.97 66.04) (width 0.25) (layer F.Cu) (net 19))
 (segment (start 138.43 50.8) (end 138.43 66.04) (width 0.25) (layer F.Cu) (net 17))
 (segment (start 135.89 50.8) (end 135.89 66.04) (width 0.25) (layer F.Cu) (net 15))
 (segment (start 133.35 50.8) (end 133.35 66.04) (width 0.25) (layer F.Cu) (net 13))
 (segment (start 140.97 143.51) (end 140.97 167.64) (width 0.25) (layer B.Cu) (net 40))
 (segment (start 135.89 138.43) (end 140.97 143.51) (width 0.25) (layer B.Cu) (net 40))
 (segment (start 134.764999 83.675001) (end 134.764999 119.235001) (width 0.25) (layer B.Cu) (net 20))
 (segment (start 140.97 77.47) (end 134.764999 83.675001) (width 0.25) (layer B.Cu) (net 20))
 (segment (start 135.89 120.360002) (end 135.89 120.65) (width 0.25) (layer B.Cu) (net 20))
 (segment (start 134.764999 119.235001) (end 135.89 120.360002) (width 0.25) (layer B.Cu) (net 20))
 (segment (start 137.015001 121.775001) (end 137.015001 127.144999) (width 0.25) (layer B.Cu) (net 20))
 (segment (start 135.89 120.65) (end 137.015001 121.775001) (width 0.25) (layer B.Cu) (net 20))
 (segment (start 134.764999 150.004999) (end 135.89 151.13) (width 0.25) (layer B.Cu) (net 20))
 (segment (start 134.764999 129.395001) (end 134.764999 150.004999) (width 0.25) (layer B.Cu) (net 20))
 (segment (start 137.015001 127.144999) (end 134.764999 129.395001) (width 0.25) (layer B.Cu) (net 20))
 (segment (start 138.43 153.67) (end 138.43 167.64) (width 0.25) (layer F.Cu) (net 20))
 (segment (start 135.89 151.13) (end 138.43 153.67) (width 0.25) (layer F.Cu) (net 20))
 (segment (start 138.43 77.47) (end 133.35 82.55) (width 0.25) (layer B.Cu) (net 18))
 (segment (start 133.35 120.65) (end 135.89 123.19) (width 0.25) (layer B.Cu) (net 18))
 (segment (start 133.35 82.55) (end 133.35 120.65) (width 0.25) (layer B.Cu) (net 18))
 (segment (start 135.89 123.19) (end 133.35 125.73) (width 0.25) (layer B.Cu) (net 18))
 (segment (start 133.35 125.73) (end 133.35 151.13) (width 0.25) (layer B.Cu) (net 18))
 (segment (start 133.35 151.13) (end 135.89 153.67) (width 0.25) (layer B.Cu) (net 18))
 (segment (start 137.015001 154.795001) (end 137.015001 158.894999) (width 0.25) (layer F.Cu) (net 18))
 (segment (start 135.89 153.67) (end 137.015001 154.795001) (width 0.25) (layer F.Cu) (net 18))
 (segment (start 135.89 160.02) (end 135.89 167.64) (width 0.25) (layer F.Cu) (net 18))
 (segment (start 137.015001 158.894999) (end 135.89 160.02) (width 0.25) (layer F.Cu) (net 18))
 (segment (start 130.81 118.11) (end 128.27 120.65) (width 0.25) (layer B.Cu) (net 14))
 (segment (start 130.81 80.01) (end 130.81 118.11) (width 0.25) (layer B.Cu) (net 14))
 (segment (start 133.35 77.47) (end 130.81 80.01) (width 0.25) (layer B.Cu) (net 14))
 (segment (start 128.27 120.65) (end 127 121.92) (width 0.25) (layer B.Cu) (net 14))
 (segment (start 127 121.92) (end 127 128.27) (width 0.25) (layer B.Cu) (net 14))
 (segment (start 129.395001 150.004999) (end 128.27 151.13) (width 0.25) (layer B.Cu) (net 14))
 (segment (start 129.395001 130.665001) (end 129.395001 150.004999) (width 0.25) (layer B.Cu) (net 14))
 (segment (start 127 128.27) (end 129.395001 130.665001) (width 0.25) (layer B.Cu) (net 14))
 (segment (start 133.35 156.21) (end 133.35 167.64) (width 0.25) (layer F.Cu) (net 14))
 (segment (start 128.27 151.13) (end 133.35 156.21) (width 0.25) (layer F.Cu) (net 14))
 (segment (start 135.89 77.47) (end 132.08 81.28) (width 0.25) (layer B.Cu) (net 16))
 (segment (start 132.08 81.28) (end 132.08 119.38) (width 0.25) (layer B.Cu) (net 16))
 (segment (start 132.08 119.38) (end 128.27 123.19) (width 0.25) (layer B.Cu) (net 16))
 (segment (start 128.27 123.19) (end 130.81 125.73) (width 0.25) (layer B.Cu) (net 16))
 (segment (start 130.81 151.13) (end 128.27 153.67) (width 0.25) (layer B.Cu) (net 16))
 (segment (start 130.81 125.73) (end 130.81 151.13) (width 0.25) (layer B.Cu) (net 16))
 (segment (start 130.81 156.21) (end 130.81 167.64) (width 0.25) (layer F.Cu) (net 16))
 (segment (start 128.27 153.67) (end 130.81 156.21) (width 0.25) (layer F.Cu) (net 16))
 (segment (start 134.764999 106.824999) (end 121.775001 106.824999) (width 0.25) (layer F.Cu) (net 42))
 (segment (start 135.89 107.95) (end 134.764999 106.824999) (width 0.25) (layer F.Cu) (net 42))
 (segment (start 121.775001 106.824999) (end 114.3 114.3) (width 0.25) (layer F.Cu) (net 42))
 (segment (start 114.3 114.3) (end 114.3 133.35) (width 0.25) (layer F.Cu) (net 42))
 (segment (start 119.38 138.43) (end 128.27 138.43) (width 0.25) (layer F.Cu) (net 42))
 (segment (start 114.3 133.35) (end 119.38 138.43) (width 0.25) (layer F.Cu) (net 42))
 (segment (start 128.27 118.11) (end 124.46 118.11) (width 0.25) (layer F.Cu) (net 28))
 (segment (start 135.89 113.03) (end 143.51 113.03) (width 0.25) (layer F.Cu) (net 25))
 (segment (start 128.27 115.57) (end 124.46 115.57) (width 0.25) (layer F.Cu) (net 29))
 (segment (start 135.89 115.57) (end 143.51 115.57) (width 0.25) (layer F.Cu) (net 26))
 (segment (start 128.27 113.03) (end 124.46 113.03) (width 0.25) (layer F.Cu) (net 30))
 (segment (start 135.89 118.11) (end 143.51 118.11) (width 0.25) (layer F.Cu) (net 27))
 (segment (start 128.27 110.49) (end 124.46 110.49) (width 0.25) (layer F.Cu) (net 31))
 (segment (start 129.54 106.68) (end 128.27 107.95) (width 0.25) (layer B.Cu) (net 12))
 (segment (start 129.54 78.74) (end 129.54 106.68) (width 0.25) (layer B.Cu) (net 12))
 (segment (start 130.81 77.47) (end 129.54 78.74) (width 0.25) (layer B.Cu) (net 12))
 (segment (start 137.16 140.97) (end 140.97 137.16) (width 0.25) (layer F.Cu) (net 41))
 (segment (start 135.89 140.97) (end 137.16 140.97) (width 0.25) (layer F.Cu) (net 41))
 (segment (start 143.51 137.16) (end 143.51 140.97) (width 0.25) (layer F.Cu) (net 32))
 (segment (start 113.03 96.52) (end 107.95 101.6) (width 0.25) (layer F.Cu) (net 22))
 (segment (start 113.03 93.98) (end 113.03 96.52) (width 0.25) (layer F.Cu) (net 22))
 (segment (start 106.68 93.98) (end 106.68 96.52) (width 0.25) (layer F.Cu) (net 23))
 (segment (start 106.68 96.52) (end 105.41 97.79) (width 0.25) (layer F.Cu) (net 23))
 (segment (start 105.41 97.79) (end 105.41 101.6) (width 0.25) (layer F.Cu) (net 23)))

